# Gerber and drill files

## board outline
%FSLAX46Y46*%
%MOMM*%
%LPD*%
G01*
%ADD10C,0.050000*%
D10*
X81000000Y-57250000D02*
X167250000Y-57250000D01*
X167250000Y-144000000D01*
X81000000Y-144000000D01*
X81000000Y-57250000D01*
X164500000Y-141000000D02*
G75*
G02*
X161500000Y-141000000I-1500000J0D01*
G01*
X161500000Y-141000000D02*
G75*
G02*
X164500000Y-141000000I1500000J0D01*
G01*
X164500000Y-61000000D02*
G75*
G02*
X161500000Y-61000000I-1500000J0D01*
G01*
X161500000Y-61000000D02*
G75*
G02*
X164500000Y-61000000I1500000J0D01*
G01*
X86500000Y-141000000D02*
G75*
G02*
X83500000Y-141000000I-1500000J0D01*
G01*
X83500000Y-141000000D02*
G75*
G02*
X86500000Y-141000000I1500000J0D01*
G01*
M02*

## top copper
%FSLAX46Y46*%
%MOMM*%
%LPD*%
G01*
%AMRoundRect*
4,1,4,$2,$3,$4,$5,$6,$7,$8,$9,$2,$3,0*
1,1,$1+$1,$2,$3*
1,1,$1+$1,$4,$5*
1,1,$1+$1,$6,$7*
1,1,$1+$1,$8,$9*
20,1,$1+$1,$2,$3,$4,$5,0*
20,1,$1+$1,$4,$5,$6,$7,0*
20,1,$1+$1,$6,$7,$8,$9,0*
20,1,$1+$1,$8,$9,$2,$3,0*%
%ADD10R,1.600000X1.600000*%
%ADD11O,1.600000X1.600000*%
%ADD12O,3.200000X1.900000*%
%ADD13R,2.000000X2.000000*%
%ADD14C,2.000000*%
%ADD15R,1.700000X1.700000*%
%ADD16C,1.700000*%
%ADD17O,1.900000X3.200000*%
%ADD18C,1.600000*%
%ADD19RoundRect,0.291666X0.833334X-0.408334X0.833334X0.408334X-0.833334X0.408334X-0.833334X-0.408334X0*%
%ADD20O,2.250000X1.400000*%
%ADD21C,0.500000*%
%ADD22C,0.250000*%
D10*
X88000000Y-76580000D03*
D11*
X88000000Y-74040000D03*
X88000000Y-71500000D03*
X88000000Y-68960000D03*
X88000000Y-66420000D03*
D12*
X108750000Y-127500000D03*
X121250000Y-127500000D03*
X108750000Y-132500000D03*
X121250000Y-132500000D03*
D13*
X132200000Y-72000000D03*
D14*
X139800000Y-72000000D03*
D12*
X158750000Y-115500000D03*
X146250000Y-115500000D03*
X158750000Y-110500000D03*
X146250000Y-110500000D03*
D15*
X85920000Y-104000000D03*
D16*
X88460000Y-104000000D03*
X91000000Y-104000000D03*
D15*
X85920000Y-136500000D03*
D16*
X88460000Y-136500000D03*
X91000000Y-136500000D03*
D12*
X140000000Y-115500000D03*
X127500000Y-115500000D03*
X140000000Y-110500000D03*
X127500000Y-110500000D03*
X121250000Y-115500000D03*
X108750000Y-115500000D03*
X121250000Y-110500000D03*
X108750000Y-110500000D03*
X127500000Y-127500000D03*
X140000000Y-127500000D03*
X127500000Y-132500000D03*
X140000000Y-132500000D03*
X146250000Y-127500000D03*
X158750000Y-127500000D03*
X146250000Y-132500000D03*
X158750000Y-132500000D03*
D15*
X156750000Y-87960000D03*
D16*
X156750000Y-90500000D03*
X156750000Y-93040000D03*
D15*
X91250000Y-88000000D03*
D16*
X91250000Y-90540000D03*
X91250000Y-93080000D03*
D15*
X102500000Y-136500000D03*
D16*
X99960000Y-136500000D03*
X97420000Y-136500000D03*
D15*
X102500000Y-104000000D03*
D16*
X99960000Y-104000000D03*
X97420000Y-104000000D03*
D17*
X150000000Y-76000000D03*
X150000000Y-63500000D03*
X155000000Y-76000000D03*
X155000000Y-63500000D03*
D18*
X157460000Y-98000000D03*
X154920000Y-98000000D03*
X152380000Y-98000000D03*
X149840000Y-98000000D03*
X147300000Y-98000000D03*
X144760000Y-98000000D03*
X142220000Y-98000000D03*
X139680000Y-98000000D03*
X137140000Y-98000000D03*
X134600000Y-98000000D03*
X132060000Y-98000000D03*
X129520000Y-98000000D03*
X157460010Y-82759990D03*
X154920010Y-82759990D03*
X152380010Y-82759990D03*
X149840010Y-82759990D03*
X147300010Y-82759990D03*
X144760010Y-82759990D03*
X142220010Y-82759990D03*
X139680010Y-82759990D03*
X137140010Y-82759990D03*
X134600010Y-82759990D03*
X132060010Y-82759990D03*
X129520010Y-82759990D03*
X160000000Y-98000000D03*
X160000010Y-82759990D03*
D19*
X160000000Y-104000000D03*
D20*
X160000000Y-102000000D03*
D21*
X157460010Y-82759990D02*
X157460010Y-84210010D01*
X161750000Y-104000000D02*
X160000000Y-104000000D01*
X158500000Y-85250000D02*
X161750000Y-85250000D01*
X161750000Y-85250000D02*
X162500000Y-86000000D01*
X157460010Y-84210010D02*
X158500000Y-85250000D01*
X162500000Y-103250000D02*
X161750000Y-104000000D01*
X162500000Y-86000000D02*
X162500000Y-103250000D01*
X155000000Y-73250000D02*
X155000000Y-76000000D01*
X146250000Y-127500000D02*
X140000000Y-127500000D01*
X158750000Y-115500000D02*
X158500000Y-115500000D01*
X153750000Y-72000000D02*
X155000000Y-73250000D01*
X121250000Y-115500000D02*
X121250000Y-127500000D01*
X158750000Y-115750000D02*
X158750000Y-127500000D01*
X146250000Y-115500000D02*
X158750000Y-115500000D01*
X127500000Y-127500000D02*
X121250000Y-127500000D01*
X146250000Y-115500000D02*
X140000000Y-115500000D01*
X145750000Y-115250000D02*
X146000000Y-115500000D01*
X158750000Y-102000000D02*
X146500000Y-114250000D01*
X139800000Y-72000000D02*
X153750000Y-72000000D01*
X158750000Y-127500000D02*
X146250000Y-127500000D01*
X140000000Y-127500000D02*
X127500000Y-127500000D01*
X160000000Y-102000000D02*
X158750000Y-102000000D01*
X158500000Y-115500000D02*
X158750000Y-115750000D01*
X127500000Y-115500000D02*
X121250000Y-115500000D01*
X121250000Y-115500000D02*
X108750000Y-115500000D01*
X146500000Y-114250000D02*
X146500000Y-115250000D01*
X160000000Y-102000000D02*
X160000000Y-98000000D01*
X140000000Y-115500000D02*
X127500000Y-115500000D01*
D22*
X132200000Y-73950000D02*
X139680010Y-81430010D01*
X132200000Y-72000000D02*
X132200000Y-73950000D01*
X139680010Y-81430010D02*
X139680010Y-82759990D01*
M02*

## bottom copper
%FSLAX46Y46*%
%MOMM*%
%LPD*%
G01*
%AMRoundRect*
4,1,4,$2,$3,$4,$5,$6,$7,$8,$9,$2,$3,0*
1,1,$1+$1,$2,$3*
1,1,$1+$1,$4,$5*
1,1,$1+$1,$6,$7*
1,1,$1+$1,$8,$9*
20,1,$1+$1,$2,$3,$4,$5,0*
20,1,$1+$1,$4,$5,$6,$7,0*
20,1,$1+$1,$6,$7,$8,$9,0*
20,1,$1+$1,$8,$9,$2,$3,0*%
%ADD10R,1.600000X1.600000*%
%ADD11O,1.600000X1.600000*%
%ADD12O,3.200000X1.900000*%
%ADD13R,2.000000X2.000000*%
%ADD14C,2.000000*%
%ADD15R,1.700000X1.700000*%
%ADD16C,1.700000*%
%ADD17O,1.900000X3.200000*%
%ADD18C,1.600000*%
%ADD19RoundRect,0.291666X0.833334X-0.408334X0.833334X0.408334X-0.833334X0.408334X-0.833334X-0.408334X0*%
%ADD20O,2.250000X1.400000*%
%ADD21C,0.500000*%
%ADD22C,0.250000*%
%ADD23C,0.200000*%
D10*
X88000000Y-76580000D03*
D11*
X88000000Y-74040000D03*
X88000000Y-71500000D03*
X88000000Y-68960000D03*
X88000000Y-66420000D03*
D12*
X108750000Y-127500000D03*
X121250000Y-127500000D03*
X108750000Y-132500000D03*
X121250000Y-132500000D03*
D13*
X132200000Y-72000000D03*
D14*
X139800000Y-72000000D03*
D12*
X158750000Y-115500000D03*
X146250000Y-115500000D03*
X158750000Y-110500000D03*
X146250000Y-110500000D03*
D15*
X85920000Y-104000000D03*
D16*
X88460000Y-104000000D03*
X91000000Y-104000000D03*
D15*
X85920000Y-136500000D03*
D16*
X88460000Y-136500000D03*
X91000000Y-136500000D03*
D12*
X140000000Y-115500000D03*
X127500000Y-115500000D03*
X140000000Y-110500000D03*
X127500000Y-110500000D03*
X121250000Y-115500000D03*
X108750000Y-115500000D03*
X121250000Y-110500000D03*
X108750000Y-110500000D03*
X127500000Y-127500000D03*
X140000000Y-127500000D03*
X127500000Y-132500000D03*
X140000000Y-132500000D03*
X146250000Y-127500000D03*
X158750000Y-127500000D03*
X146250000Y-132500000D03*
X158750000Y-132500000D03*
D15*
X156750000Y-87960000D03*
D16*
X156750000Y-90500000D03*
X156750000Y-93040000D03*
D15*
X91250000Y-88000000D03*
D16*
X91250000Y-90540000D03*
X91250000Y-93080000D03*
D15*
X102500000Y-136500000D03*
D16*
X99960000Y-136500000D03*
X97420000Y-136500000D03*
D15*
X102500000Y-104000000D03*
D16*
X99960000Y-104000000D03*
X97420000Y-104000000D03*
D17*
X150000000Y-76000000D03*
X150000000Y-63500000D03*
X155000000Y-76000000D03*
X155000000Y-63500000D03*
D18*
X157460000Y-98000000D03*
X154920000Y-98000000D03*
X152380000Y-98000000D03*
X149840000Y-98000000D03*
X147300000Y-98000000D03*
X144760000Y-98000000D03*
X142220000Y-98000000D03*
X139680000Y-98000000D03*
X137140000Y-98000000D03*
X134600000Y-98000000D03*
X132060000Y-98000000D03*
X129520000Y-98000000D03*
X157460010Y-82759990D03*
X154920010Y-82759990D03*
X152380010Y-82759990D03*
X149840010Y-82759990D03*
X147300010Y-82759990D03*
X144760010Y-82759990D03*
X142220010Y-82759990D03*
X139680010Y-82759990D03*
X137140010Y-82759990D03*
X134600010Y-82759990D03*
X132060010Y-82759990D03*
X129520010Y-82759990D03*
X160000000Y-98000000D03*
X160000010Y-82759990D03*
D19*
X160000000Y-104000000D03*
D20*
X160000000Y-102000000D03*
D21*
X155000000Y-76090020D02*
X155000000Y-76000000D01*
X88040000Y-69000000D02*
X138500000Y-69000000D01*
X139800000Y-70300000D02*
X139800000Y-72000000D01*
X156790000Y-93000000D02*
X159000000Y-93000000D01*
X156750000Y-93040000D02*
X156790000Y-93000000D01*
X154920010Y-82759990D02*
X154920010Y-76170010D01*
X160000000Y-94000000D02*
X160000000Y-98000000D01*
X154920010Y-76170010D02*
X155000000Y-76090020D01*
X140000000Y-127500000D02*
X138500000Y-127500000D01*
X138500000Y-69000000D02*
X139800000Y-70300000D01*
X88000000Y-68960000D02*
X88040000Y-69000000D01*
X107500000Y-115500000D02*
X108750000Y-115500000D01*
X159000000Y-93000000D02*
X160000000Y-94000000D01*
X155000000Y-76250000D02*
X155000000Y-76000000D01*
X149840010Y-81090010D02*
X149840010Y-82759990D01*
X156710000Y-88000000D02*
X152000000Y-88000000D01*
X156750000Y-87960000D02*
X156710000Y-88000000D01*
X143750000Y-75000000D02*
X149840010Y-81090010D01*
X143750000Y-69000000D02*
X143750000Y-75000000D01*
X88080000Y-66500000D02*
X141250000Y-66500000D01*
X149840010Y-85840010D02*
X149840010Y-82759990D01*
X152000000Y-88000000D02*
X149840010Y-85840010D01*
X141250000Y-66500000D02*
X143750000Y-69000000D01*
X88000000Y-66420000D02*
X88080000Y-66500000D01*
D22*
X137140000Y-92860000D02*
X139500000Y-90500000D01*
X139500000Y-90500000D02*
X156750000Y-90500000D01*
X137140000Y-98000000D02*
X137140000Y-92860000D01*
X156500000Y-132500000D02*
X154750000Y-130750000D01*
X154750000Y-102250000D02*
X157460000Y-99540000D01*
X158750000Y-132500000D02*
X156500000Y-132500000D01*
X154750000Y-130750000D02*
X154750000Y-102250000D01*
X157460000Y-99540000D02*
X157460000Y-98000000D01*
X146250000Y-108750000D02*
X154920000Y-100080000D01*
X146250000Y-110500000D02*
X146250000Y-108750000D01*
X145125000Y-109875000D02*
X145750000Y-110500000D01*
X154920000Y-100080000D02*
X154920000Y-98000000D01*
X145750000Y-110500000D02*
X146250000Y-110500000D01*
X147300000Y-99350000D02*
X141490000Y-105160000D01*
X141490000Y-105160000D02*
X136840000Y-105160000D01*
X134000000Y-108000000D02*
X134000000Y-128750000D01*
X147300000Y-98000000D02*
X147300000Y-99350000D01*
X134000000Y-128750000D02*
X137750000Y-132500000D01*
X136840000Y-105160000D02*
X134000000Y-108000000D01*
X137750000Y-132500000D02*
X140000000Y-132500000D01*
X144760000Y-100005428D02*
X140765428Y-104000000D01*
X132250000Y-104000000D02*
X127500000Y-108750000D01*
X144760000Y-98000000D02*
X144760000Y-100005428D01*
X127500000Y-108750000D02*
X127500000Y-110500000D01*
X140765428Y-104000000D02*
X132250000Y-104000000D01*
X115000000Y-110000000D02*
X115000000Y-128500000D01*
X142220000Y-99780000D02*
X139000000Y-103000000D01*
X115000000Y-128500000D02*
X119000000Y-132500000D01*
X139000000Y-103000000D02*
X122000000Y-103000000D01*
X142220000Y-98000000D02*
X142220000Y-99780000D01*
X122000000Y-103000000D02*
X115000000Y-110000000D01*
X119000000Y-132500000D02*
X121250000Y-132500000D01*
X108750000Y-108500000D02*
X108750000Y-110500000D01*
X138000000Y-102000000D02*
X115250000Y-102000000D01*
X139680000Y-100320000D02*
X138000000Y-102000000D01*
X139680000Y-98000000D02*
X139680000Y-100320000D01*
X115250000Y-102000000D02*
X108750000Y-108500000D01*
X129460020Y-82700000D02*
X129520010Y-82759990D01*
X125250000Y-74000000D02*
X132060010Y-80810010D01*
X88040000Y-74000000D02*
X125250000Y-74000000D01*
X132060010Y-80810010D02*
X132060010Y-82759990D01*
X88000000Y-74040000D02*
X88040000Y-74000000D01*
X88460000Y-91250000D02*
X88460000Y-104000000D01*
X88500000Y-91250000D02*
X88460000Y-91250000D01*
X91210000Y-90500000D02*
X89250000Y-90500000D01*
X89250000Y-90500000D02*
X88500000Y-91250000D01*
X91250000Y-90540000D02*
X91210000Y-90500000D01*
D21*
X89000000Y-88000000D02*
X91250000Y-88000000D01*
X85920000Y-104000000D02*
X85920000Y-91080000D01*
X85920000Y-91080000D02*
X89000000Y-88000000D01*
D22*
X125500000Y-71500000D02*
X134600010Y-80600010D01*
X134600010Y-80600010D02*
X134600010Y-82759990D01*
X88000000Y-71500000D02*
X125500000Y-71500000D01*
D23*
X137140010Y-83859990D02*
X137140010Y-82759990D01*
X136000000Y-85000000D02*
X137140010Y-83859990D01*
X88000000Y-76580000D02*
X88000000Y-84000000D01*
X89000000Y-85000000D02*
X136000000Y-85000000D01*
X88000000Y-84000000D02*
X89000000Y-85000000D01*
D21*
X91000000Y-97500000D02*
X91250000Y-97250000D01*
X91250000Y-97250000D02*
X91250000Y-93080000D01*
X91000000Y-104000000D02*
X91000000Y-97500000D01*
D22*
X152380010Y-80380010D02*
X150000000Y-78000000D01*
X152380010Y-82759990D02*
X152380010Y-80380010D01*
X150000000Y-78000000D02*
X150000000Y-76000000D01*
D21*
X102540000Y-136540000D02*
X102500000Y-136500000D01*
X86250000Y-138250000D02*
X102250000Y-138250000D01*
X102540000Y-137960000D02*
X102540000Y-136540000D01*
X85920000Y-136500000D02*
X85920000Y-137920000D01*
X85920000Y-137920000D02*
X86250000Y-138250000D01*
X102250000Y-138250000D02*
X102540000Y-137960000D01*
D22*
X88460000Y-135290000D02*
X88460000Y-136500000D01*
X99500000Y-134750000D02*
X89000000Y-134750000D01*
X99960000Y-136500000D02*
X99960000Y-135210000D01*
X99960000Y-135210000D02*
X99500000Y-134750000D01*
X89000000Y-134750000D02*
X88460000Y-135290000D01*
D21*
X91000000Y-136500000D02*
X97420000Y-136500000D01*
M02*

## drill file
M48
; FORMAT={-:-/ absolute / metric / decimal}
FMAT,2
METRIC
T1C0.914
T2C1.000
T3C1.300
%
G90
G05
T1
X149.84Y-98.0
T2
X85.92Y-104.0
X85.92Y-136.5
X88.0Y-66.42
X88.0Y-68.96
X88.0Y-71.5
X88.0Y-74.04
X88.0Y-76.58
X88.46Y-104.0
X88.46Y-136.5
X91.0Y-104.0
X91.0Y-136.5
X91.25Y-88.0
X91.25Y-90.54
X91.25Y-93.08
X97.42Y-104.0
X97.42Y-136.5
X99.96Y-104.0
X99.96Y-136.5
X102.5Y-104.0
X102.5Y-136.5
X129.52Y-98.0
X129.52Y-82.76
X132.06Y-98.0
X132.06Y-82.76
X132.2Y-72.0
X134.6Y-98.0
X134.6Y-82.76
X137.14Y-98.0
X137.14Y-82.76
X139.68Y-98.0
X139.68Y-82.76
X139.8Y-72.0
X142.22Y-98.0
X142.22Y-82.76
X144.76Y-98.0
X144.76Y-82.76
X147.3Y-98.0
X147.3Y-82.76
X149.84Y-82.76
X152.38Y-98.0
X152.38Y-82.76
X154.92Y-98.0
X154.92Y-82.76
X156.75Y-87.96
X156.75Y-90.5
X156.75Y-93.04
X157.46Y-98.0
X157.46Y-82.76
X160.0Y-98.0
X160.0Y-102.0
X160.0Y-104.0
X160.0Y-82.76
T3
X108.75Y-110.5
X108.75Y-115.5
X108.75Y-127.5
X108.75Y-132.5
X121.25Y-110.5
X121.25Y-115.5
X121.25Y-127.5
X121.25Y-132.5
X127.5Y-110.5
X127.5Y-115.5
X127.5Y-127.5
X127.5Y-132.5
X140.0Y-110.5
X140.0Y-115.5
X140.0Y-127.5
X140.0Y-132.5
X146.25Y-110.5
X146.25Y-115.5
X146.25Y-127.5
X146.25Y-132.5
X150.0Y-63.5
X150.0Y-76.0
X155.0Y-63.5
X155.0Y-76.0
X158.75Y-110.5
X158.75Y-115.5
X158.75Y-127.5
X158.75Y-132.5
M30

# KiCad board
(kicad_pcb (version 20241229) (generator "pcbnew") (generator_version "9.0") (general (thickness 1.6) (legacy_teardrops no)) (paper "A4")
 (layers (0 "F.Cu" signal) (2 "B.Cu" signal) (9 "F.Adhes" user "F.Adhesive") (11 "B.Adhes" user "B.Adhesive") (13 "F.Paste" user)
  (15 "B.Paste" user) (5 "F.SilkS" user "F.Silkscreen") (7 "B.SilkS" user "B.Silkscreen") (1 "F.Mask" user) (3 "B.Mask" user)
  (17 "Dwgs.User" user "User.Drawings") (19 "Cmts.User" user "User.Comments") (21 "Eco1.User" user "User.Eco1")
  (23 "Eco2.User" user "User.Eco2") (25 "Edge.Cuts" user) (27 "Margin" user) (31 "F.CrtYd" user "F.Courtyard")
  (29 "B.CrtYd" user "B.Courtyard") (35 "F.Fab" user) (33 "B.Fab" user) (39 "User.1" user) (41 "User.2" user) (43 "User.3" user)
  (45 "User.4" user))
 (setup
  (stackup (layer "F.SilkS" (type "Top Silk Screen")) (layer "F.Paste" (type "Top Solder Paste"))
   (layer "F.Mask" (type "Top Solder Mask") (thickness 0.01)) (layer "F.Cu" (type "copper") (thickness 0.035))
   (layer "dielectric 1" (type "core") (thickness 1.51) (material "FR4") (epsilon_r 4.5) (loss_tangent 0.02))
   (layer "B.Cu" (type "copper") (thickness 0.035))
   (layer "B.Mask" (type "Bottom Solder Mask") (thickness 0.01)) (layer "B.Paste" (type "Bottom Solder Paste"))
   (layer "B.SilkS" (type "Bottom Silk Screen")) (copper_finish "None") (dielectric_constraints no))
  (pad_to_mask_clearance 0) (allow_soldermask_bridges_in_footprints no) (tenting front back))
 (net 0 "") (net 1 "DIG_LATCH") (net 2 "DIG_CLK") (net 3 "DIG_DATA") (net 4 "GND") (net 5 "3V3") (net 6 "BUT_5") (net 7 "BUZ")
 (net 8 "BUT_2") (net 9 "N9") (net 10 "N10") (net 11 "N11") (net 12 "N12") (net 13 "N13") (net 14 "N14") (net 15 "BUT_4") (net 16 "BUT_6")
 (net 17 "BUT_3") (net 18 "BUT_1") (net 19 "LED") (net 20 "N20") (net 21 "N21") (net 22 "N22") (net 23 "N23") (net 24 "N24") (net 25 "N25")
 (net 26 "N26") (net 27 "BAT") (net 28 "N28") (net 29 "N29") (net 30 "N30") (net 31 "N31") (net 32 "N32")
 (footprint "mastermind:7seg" (layer "F.Cu") (at 94.5 68)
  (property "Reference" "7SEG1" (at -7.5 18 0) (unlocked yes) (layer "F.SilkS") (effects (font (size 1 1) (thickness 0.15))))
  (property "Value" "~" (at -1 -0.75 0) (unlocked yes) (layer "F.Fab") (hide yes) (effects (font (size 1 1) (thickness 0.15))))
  (pad "1" thru_hole rect (at -6.5 8.58 180) (size 1.6 1.6) (drill 1) (layers "*.Cu" "*.Mask") (remove_unused_layers no) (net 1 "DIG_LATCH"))
  (pad "2" thru_hole oval (at -6.5 6.04 180) (size 1.6 1.6) (drill 1) (layers "*.Cu" "*.Mask") (remove_unused_layers no) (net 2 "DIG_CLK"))
  (pad "3" thru_hole oval (at -6.5 3.5 180) (size 1.6 1.6) (drill 1) (layers "*.Cu" "*.Mask") (remove_unused_layers no) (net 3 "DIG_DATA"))
  (pad "4" thru_hole oval (at -6.5 0.96 180) (size 1.6 1.6) (drill 1) (layers "*.Cu" "*.Mask") (remove_unused_layers no) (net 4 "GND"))
  (pad "5" thru_hole oval (at -6.5 -1.58 180) (size 1.6 1.6) (drill 1) (layers "*.Cu" "*.Mask") (remove_unused_layers no) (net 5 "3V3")))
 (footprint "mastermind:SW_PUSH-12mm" (layer "F.Cu") (at 108.75 127.5)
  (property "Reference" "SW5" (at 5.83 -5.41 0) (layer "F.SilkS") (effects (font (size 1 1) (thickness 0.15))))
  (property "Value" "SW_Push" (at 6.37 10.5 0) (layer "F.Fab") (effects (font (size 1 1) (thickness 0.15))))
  (pad "1" thru_hole oval (at 0 0) (size 3.2 1.9) (drill 1.3) (layers "*.Cu" "*.Mask") (remove_unused_layers no) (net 4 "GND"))
  (pad "1" thru_hole oval (at 12.5 0) (size 3.2 1.9) (drill 1.3) (layers "*.Cu" "*.Mask") (remove_unused_layers no) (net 4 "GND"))
  (pad "2" thru_hole oval (at 0 5) (size 3.2 1.9) (drill 1.3) (layers "*.Cu" "*.Mask") (remove_unused_layers no) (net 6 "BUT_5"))
  (pad "2" thru_hole oval (at 12.5 5) (size 3.2 1.9) (drill 1.3) (layers "*.Cu" "*.Mask") (remove_unused_layers no) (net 6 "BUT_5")))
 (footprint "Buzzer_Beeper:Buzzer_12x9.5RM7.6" (layer "F.Cu") (at 132.2 72)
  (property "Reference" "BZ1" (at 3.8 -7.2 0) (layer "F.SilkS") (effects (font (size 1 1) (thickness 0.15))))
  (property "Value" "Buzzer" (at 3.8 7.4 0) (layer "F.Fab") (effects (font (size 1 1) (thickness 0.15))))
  (pad "1" thru_hole rect (at 0 0) (size 2 2) (drill 1) (layers "*.Cu" "*.Mask") (remove_unused_layers no) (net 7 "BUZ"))
  (pad "2" thru_hole circle (at 7.6 0) (size 2 2) (drill 1) (layers "*.Cu" "*.Mask") (remove_unused_layers no) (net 4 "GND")))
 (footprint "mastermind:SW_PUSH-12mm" (layer "F.Cu") (at 158.75 115.5 180)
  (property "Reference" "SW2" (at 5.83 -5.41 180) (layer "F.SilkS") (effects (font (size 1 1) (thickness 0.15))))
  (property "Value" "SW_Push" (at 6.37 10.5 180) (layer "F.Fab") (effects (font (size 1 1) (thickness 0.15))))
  (pad "1" thru_hole oval (at 0 0 180) (size 3.2 1.9) (drill 1.3) (layers "*.Cu" "*.Mask") (remove_unused_layers no) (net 4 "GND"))
  (pad "1" thru_hole oval (at 12.5 0 180) (size 3.2 1.9) (drill 1.3) (layers "*.Cu" "*.Mask") (remove_unused_layers no) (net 4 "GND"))
  (pad "2" thru_hole oval (at 0 5 180) (size 3.2 1.9) (drill 1.3) (layers "*.Cu" "*.Mask") (remove_unused_layers no) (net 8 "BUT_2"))
  (pad "2" thru_hole oval (at 12.5 5 180) (size 3.2 1.9) (drill 1.3) (layers "*.Cu" "*.Mask") (remove_unused_layers no) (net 8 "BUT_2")))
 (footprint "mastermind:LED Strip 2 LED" (layer "F.Cu") (at 88.17 111.25 90)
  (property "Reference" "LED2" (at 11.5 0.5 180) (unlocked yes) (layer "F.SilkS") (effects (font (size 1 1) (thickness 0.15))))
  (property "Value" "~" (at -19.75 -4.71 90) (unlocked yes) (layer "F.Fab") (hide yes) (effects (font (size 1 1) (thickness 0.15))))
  (pad "1" thru_hole rect (at 7.25 -2.25 90) (size 1.7 1.7) (drill 1) (layers "*.Cu" "*.Mask") (remove_unused_layers no) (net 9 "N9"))
  (pad "2" thru_hole circle (at 7.25 0.29 90) (size 1.7 1.7) (drill 1) (layers "*.Cu" "*.Mask") (remove_unused_layers no) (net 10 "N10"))
  (pad "3" thru_hole circle (at 7.25 2.83 90) (size 1.7 1.7) (drill 1) (layers "*.Cu" "*.Mask") (remove_unused_layers no) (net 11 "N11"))
  (pad "4" thru_hole rect (at -25.25 -2.25 90) (size 1.7 1.7) (drill 1) (layers "*.Cu" "*.Mask") (remove_unused_layers no) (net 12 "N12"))
  (pad "5" thru_hole circle (at -25.25 0.29 90) (size 1.7 1.7) (drill 1) (layers "*.Cu" "*.Mask") (remove_unused_layers no) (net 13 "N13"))
  (pad "6" thru_hole circle (at -25.25 2.83 90) (size 1.7 1.7) (drill 1) (layers "*.Cu" "*.Mask") (remove_unused_layers no) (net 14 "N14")))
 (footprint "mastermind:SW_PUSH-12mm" (layer "F.Cu") (at 140 115.5 180)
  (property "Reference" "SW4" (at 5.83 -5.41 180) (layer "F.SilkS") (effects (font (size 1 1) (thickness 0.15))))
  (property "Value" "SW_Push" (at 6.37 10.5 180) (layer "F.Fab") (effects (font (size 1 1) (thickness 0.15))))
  (pad "1" thru_hole oval (at 0 0 180) (size 3.2 1.9) (drill 1.3) (layers "*.Cu" "*.Mask") (remove_unused_layers no) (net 4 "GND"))
  (pad "1" thru_hole oval (at 12.5 0 180) (size 3.2 1.9) (drill 1.3) (layers "*.Cu" "*.Mask") (remove_unused_layers no) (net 4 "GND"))
  (pad "2" thru_hole oval (at 0 5 180) (size 3.2 1.9) (drill 1.3) (layers "*.Cu" "*.Mask") (remove_unused_layers no) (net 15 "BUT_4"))
  (pad "2" thru_hole oval (at 12.5 5 180) (size 3.2 1.9) (drill 1.3) (layers "*.Cu" "*.Mask") (remove_unused_layers no) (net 15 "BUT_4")))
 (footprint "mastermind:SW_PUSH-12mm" (layer "F.Cu") (at 121.25 115.5 180)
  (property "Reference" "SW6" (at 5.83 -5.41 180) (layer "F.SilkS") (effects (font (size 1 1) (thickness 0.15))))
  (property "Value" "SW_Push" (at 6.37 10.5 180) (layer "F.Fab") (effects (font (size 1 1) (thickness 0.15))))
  (pad "1" thru_hole oval (at 0 0 180) (size 3.2 1.9) (drill 1.3) (layers "*.Cu" "*.Mask") (remove_unused_layers no) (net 4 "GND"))
  (pad "1" thru_hole oval (at 12.5 0 180) (size 3.2 1.9) (drill 1.3) (layers "*.Cu" "*.Mask") (remove_unused_layers no) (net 4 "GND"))
  (pad "2" thru_hole oval (at 0 5 180) (size 3.2 1.9) (drill 1.3) (layers "*.Cu" "*.Mask") (remove_unused_layers no) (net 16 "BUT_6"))
  (pad "2" thru_hole oval (at 12.5 5 180) (size 3.2 1.9) (drill 1.3) (layers "*.Cu" "*.Mask") (remove_unused_layers no) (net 16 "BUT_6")))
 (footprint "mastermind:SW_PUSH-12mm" (layer "F.Cu") (at 127.5 127.5)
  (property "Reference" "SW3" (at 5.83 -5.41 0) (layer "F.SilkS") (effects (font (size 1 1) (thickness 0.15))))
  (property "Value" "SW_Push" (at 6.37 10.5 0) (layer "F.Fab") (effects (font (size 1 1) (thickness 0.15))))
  (pad "1" thru_hole oval (at 0 0) (size 3.2 1.9) (drill 1.3) (layers "*.Cu" "*.Mask") (remove_unused_layers no) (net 4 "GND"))
  (pad "1" thru_hole oval (at 12.5 0) (size 3.2 1.9) (drill 1.3) (layers "*.Cu" "*.Mask") (remove_unused_layers no) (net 4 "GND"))
  (pad "2" thru_hole oval (at 0 5) (size 3.2 1.9) (drill 1.3) (layers "*.Cu" "*.Mask") (remove_unused_layers no) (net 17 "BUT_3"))
  (pad "2" thru_hole oval (at 12.5 5) (size 3.2 1.9) (drill 1.3) (layers "*.Cu" "*.Mask") (remove_unused_layers no) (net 17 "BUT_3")))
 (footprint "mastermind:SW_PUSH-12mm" (layer "F.Cu") (at 146.25 127.5)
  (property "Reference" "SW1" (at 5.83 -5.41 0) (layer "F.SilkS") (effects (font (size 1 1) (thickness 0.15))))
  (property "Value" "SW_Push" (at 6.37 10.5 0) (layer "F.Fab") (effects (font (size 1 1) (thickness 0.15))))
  (pad "1" thru_hole oval (at 0 0) (size 3.2 1.9) (drill 1.3) (layers "*.Cu" "*.Mask") (remove_unused_layers no) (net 4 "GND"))
  (pad "1" thru_hole oval (at 12.5 0) (size 3.2 1.9) (drill 1.3) (layers "*.Cu" "*.Mask") (remove_unused_layers no) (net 4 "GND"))
  (pad "2" thru_hole oval (at 0 5) (size 3.2 1.9) (drill 1.3) (layers "*.Cu" "*.Mask") (remove_unused_layers no) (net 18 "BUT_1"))
  (pad "2" thru_hole oval (at 12.5 5) (size 3.2 1.9) (drill 1.3) (layers "*.Cu" "*.Mask") (remove_unused_layers no) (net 18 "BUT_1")))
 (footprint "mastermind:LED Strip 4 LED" (layer "F.Cu") (at 115.5 90.25)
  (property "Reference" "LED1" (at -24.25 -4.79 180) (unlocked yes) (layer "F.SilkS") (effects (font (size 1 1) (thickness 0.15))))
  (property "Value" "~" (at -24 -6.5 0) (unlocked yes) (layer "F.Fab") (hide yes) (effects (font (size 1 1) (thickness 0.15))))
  (pad "1" thru_hole rect (at 41.25 -2.29) (size 1.7 1.7) (drill 1) (layers "*.Cu" "*.Mask") (remove_unused_layers no) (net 5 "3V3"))
  (pad "2" thru_hole circle (at 41.25 0.25) (size 1.7 1.7) (drill 1) (layers "*.Cu" "*.Mask") (remove_unused_layers no) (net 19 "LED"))
  (pad "3" thru_hole circle (at 41.25 2.79) (size 1.7 1.7) (drill 1) (layers "*.Cu" "*.Mask") (remove_unused_layers no) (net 4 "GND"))
  (pad "4" thru_hole rect (at -24.25 -2.25) (size 1.7 1.7) (drill 1) (layers "*.Cu" "*.Mask") (remove_unused_layers no) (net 9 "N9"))
  (pad "5" thru_hole circle (at -24.25 0.29) (size 1.7 1.7) (drill 1) (layers "*.Cu" "*.Mask") (remove_unused_layers no) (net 10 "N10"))
  (pad "6" thru_hole circle (at -24.25 2.83) (size 1.7 1.7) (drill 1) (layers "*.Cu" "*.Mask") (remove_unused_layers no) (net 11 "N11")))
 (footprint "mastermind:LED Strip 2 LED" (layer "F.Cu") (at 100.25 129.25 -90)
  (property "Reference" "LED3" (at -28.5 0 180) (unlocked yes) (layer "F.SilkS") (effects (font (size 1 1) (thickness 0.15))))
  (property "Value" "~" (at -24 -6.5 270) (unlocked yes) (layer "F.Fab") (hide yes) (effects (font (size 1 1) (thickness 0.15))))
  (pad "1" thru_hole rect (at 7.25 -2.25 270) (size 1.7 1.7) (drill 1) (layers "*.Cu" "*.Mask") (remove_unused_layers no) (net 12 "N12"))
  (pad "2" thru_hole circle (at 7.25 0.29 270) (size 1.7 1.7) (drill 1) (layers "*.Cu" "*.Mask") (remove_unused_layers no) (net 13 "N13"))
  (pad "3" thru_hole circle (at 7.25 2.83 270) (size 1.7 1.7) (drill 1) (layers "*.Cu" "*.Mask") (remove_unused_layers no) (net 14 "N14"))
  (pad "4" thru_hole rect (at -25.25 -2.25 270) (size 1.7 1.7) (drill 1) (layers "*.Cu" "*.Mask") (remove_unused_layers no) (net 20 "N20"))
  (pad "5" thru_hole circle (at -25.25 0.29 270) (size 1.7 1.7) (drill 1) (layers "*.Cu" "*.Mask") (remove_unused_layers no) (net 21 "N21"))
  (pad "6" thru_hole circle (at -25.25 2.83 270) (size 1.7 1.7) (drill 1) (layers "*.Cu" "*.Mask") (remove_unused_layers no) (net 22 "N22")))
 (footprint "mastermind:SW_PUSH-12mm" (layer "F.Cu") (at 150 76 90)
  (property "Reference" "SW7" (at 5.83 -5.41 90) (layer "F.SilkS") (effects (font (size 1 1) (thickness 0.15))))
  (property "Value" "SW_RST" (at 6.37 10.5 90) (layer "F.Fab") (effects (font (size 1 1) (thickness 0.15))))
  (pad "1" thru_hole oval (at 0 0 90) (size 3.2 1.9) (drill 1.3) (layers "*.Cu" "*.Mask") (remove_unused_layers no) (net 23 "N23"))
  (pad "1" thru_hole oval (at 12.5 0 90) (size 3.2 1.9) (drill 1.3) (layers "*.Cu" "*.Mask") (remove_unused_layers no) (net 23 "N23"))
  (pad "2" thru_hole oval (at 0 5 90) (size 3.2 1.9) (drill 1.3) (layers "*.Cu" "*.Mask") (remove_unused_layers no) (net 4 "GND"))
  (pad "2" thru_hole oval (at 12.5 5 90) (size 3.2 1.9) (drill 1.3) (layers "*.Cu" "*.Mask") (remove_unused_layers no) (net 4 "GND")))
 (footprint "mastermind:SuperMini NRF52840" (layer "B.Cu") (at 160 98 90)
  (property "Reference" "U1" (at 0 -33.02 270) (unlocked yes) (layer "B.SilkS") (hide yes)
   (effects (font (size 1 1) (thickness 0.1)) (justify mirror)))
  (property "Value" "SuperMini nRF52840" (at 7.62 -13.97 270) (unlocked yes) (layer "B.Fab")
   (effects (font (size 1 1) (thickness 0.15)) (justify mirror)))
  (pad "1" thru_hole circle (at 0 -2.54 180) (size 1.6 1.6) (drill 1) (layers "*.Cu" "*.Mask") (remove_unused_layers no) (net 18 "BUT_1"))
  (pad "2" thru_hole circle (at 0 -5.08 180) (size 1.6 1.6) (drill 1) (layers "*.Cu" "*.Mask") (remove_unused_layers no) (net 8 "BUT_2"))
  (pad "3" thru_hole circle (at 0 -7.62 180) (size 1.6 1.6) (drill 1) (layers "*.Cu" "*.Mask") (remove_unused_layers no) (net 4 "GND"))
  (pad "4" thru_hole circle (at 0 -10.16) (size 1.6 1.6) (drill 0.9144) (layers "*.Cu" "*.Mask") (remove_unused_layers no) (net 4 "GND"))
  (pad "5" thru_hole circle (at 0 -12.7 180) (size 1.6 1.6) (drill 1) (layers "*.Cu" "*.Mask") (remove_unused_layers no) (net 17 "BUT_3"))
  (pad "6" thru_hole circle (at 0 -15.24 180) (size 1.6 1.6) (drill 1) (layers "*.Cu" "*.Mask") (remove_unused_layers no) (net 15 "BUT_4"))
  (pad "7" thru_hole circle (at 0 -17.78 180) (size 1.6 1.6) (drill 1) (layers "*.Cu" "*.Mask") (remove_unused_layers no) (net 6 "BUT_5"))
  (pad "8" thru_hole circle (at 0 -20.32 180) (size 1.6 1.6) (drill 1) (layers "*.Cu" "*.Mask") (remove_unused_layers no) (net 16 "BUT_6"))
  (pad "9" thru_hole circle (at 0 -22.86 180) (size 1.6 1.6) (drill 1) (layers "*.Cu" "*.Mask") (remove_unused_layers no) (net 19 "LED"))
  (pad "10" thru_hole circle (at 0 -25.4 180) (size 1.6 1.6) (drill 1) (layers "*.Cu" "*.Mask") (remove_unused_layers no) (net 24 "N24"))
  (pad "11" thru_hole circle (at 0 -27.94 180) (size 1.6 1.6) (drill 1) (layers "*.Cu" "*.Mask") (remove_unused_layers no) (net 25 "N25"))
  (pad "12" thru_hole circle (at 0 -30.48 180) (size 1.6 1.6) (drill 1) (layers "*.Cu" "*.Mask") (remove_unused_layers no) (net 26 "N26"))
  (pad "13" thru_hole circle (at 15.24001 -2.53999) (size 1.6 1.6) (drill 1) (layers "*.Cu" "*.Mask") (remove_unused_layers no)
   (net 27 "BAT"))
  (pad "14" thru_hole circle (at 15.24001 -5.07999) (size 1.6 1.6) (drill 1) (layers "*.Cu" "*.Mask") (remove_unused_layers no)
   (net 4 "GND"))
  (pad "15" thru_hole circle (at 15.24001 -7.61999) (size 1.6 1.6) (drill 1) (layers "*.Cu" "*.Mask") (remove_unused_layers no)
   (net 23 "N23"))
  (pad "16" thru_hole circle (at 15.24001 -10.15999) (size 1.6 1.6) (drill 1) (layers "*.Cu" "*.Mask") (remove_unused_layers no)
   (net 5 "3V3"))
  (pad "17" thru_hole circle (at 15.24001 -12.69999) (size 1.6 1.6) (drill 1) (layers "*.Cu" "*.Mask") (remove_unused_layers no)
   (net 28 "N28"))
  (pad "18" thru_hole circle (at 15.24001 -15.23999) (size 1.6 1.6) (drill 1) (layers "*.Cu" "*.Mask") (remove_unused_layers no)
   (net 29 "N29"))
  (pad "19" thru_hole circle (at 15.24001 -17.77999) (size 1.6 1.6) (drill 1) (layers "*.Cu" "*.Mask") (remove_unused_layers no)
   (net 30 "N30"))
  (pad "20" thru_hole circle (at 15.24001 -20.31999) (size 1.6 1.6) (drill 1) (layers "*.Cu" "*.Mask") (remove_unused_layers no)
   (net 7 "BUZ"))
  (pad "21" thru_hole circle (at 15.24001 -22.85999) (size 1.6 1.6) (drill 1) (layers "*.Cu" "*.Mask") (remove_unused_layers no)
   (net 1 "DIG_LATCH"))
  (pad "22" thru_hole circle (at 15.24001 -25.39999) (size 1.6 1.6) (drill 1) (layers "*.Cu" "*.Mask") (remove_unused_layers no)
   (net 3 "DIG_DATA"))
  (pad "23" thru_hole circle (at 15.24001 -27.93999) (size 1.6 1.6) (drill 1) (layers "*.Cu" "*.Mask") (remove_unused_layers no)
   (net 2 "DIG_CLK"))
  (pad "24" thru_hole circle (at 15.24001 -30.47999 180) (size 1.6 1.6) (drill 1) (layers "*.Cu" "*.Mask") (remove_unused_layers no)
   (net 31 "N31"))
  (pad "28" thru_hole circle (at 0 0 180) (size 1.6 1.6) (drill 1) (layers "*.Cu" "*.Mask") (remove_unused_layers no) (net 4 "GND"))
  (pad "29" thru_hole circle (at 15.24001 0.00001) (size 1.6 1.6) (drill 1) (layers "*.Cu" "*.Mask") (remove_unused_layers no)
   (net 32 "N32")))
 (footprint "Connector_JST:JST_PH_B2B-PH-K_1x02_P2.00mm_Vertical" (layer "B.Cu") (at 160 104 90)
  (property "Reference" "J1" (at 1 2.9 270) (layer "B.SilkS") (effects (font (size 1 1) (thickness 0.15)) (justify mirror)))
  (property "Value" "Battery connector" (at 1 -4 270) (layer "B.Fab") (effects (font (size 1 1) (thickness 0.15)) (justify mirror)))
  (pad "1" thru_hole roundrect (at 0 0 90) (size 1.4 2.25) (drill 1) (layers "*.Cu" "*.Mask") (remove_unused_layers no)
   (roundrect_rratio 0.208333) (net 27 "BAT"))
  (pad "2" thru_hole oval (at 2 0 90) (size 1.4 2.25) (drill 1) (layers "*.Cu" "*.Mask") (remove_unused_layers no) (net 4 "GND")))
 (gr_rect (start 81 57.25) (end 167.25 144) (stroke (width 0.05) (type default)) (fill no) (layer "Edge.Cuts"))
 (gr_circle (center 163 141) (end 164.5 141) (stroke (width 0.05) (type solid)) (fill no) (layer "Edge.Cuts"))
 (gr_circle (center 163 61) (end 164.5 61) (stroke (width 0.05) (type solid)) (fill no) (layer "Edge.Cuts"))
 (gr_circle (center 85 141) (end 86.5 141) (stroke (width 0.05) (type solid)) (fill no) (layer "Edge.Cuts"))
 (segment (start 157.46001 82.75999) (end 157.46001 84.21001) (width 0.5) (layer "F.Cu") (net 27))
 (segment (start 161.75 104) (end 160 104) (width 0.5) (layer "F.Cu") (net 27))
 (segment (start 158.5 85.25) (end 161.75 85.25) (width 0.5) (layer "F.Cu") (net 27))
 (segment (start 161.75 85.25) (end 162.5 86) (width 0.5) (layer "F.Cu") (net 27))
 (segment (start 157.46001 84.21001) (end 158.5 85.25) (width 0.5) (layer "F.Cu") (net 27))
 (segment (start 162.5 103.25) (end 161.75 104) (width 0.5) (layer "F.Cu") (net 27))
 (segment (start 162.5 86) (end 162.5 103.25) (width 0.5) (layer "F.Cu") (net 27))
 (segment (start 155 73.25) (end 155 76) (width 0.5) (layer "F.Cu") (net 4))
 (segment (start 146.25 127.5) (end 140 127.5) (width 0.5) (layer "F.Cu") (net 4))
 (segment (start 158.75 115.5) (end 158.5 115.5) (width 0.5) (layer "F.Cu") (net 4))
 (segment (start 153.75 72) (end 155 73.25) (width 0.5) (layer "F.Cu") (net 4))
 (segment (start 121.25 115.5) (end 121.25 127.5) (width 0.5) (layer "F.Cu") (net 4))
 (segment (start 158.75 115.75) (end 158.75 127.5) (width 0.5) (layer "F.Cu") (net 4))
 (segment (start 146.25 115.5) (end 158.75 115.5) (width 0.5) (layer "F.Cu") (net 4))
 (segment (start 127.5 127.5) (end 121.25 127.5) (width 0.5) (layer "F.Cu") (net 4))
 (segment (start 146.25 115.5) (end 140 115.5) (width 0.5) (layer "F.Cu") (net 4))
 (segment (start 145.75 115.25) (end 146 115.5) (width 0.5) (layer "F.Cu") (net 4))
 (segment (start 158.75 102) (end 146.5 114.25) (width 0.5) (layer "F.Cu") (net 4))
 (segment (start 139.8 72) (end 153.75 72) (width 0.5) (layer "F.Cu") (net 4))
 (segment (start 158.75 127.5) (end 146.25 127.5) (width 0.5) (layer "F.Cu") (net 4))
 (segment (start 140 127.5) (end 127.5 127.5) (width 0.5) (layer "F.Cu") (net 4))
 (segment (start 160 102) (end 158.75 102) (width 0.5) (layer "F.Cu") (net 4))
 (segment (start 158.5 115.5) (end 158.75 115.75) (width 0.5) (layer "F.Cu") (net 4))
 (segment (start 127.5 115.5) (end 121.25 115.5) (width 0.5) (layer "F.Cu") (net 4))
 (segment (start 121.25 115.5) (end 108.75 115.5) (width 0.5) (layer "F.Cu") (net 4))
 (segment (start 146.5 114.25) (end 146.5 115.25) (width 0.5) (layer "F.Cu") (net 4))
 (segment (start 160 102) (end 160 98) (width 0.5) (layer "F.Cu") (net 4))
 (segment (start 140 115.5) (end 127.5 115.5) (width 0.5) (layer "F.Cu") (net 4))
 (segment (start 155 76.09002) (end 155 76) (width 0.5) (layer "B.Cu") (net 4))
 (segment (start 88.04 69) (end 138.5 69) (width 0.5) (layer "B.Cu") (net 4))
 (segment (start 139.8 70.3) (end 139.8 72) (width 0.5) (layer "B.Cu") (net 4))
 (segment (start 156.79 93) (end 159 93) (width 0.5) (layer "B.Cu") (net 4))
 (segment (start 156.75 93.04) (end 156.79 93) (width 0.5) (layer "B.Cu") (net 4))
 (segment (start 154.92001 82.75999) (end 154.92001 76.17001) (width 0.5) (layer "B.Cu") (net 4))
 (segment (start 160 94) (end 160 98) (width 0.5) (layer "B.Cu") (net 4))
 (segment (start 154.92001 76.17001) (end 155 76.09002) (width 0.5) (layer "B.Cu") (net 4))
 (segment (start 140 127.5) (end 138.5 127.5) (width 0.5) (layer "B.Cu") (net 4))
 (segment (start 138.5 69) (end 139.8 70.3) (width 0.5) (layer "B.Cu") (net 4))
 (segment (start 88 68.96) (end 88.04 69) (width 0.5) (layer "B.Cu") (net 4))
 (segment (start 107.5 115.5) (end 108.75 115.5) (width 0.5) (layer "B.Cu") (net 4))
 (segment (start 159 93) (end 160 94) (width 0.5) (layer "B.Cu") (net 4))
 (segment (start 155 76.25) (end 155 76) (width 0.5) (layer "B.Cu") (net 4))
 (segment (start 149.84001 81.09001) (end 149.84001 82.75999) (width 0.5) (layer "B.Cu") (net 5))
 (segment (start 156.71 88) (end 152 88) (width 0.5) (layer "B.Cu") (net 5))
 (segment (start 156.75 87.96) (end 156.71 88) (width 0.5) (layer "B.Cu") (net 5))
 (segment (start 143.75 75) (end 149.84001 81.09001) (width 0.5) (layer "B.Cu") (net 5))
 (segment (start 143.75 69) (end 143.75 75) (width 0.5) (layer "B.Cu") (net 5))
 (segment (start 88.08 66.5) (end 141.25 66.5) (width 0.5) (layer "B.Cu") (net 5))
 (segment (start 149.84001 85.84001) (end 149.84001 82.75999) (width 0.5) (layer "B.Cu") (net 5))
 (segment (start 152 88) (end 149.84001 85.84001) (width 0.5) (layer "B.Cu") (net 5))
 (segment (start 141.25 66.5) (end 143.75 69) (width 0.5) (layer "B.Cu") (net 5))
 (segment (start 88 66.42) (end 88.08 66.5) (width 0.5) (layer "B.Cu") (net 5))
 (segment (start 137.14 92.86) (end 139.5 90.5) (width 0.25) (layer "B.Cu") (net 19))
 (segment (start 139.5 90.5) (end 156.75 90.5) (width 0.25) (layer "B.Cu") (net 19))
 (segment (start 137.14 98) (end 137.14 92.86) (width 0.25) (layer "B.Cu") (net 19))
 (segment (start 156.5 132.5) (end 154.75 130.75) (width 0.25) (layer "B.Cu") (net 18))
 (segment (start 154.75 102.25) (end 157.46 99.54) (width 0.25) (layer "B.Cu") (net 18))
 (segment (start 158.75 132.5) (end 156.5 132.5) (width 0.25) (layer "B.Cu") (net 18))
 (segment (start 154.75 130.75) (end 154.75 102.25) (width 0.25) (layer "B.Cu") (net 18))
 (segment (start 157.46 99.54) (end 157.46 98) (width 0.25) (layer "B.Cu") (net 18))
 (segment (start 146.25 108.75) (end 154.92 100.08) (width 0.25) (layer "B.Cu") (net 8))
 (segment (start 146.25 110.5) (end 146.25 108.75) (width 0.25) (layer "B.Cu") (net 8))
 (segment (start 145.125 109.875) (end 145.75 110.5) (width 0.25) (layer "B.Cu") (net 8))
 (segment (start 154.92 100.08) (end 154.92 98) (width 0.25) (layer "B.Cu") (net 8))
 (segment (start 145.75 110.5) (end 146.25 110.5) (width 0.25) (layer "B.Cu") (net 8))
 (segment (start 147.3 99.35) (end 141.49 105.16) (width 0.25) (layer "B.Cu") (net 17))
 (segment (start 141.49 105.16) (end 136.84 105.16) (width 0.25) (layer "B.Cu") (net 17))
 (segment (start 134 108) (end 134 128.75) (width 0.25) (layer "B.Cu") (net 17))
 (segment (start 147.3 98) (end 147.3 99.35) (width 0.25) (layer "B.Cu") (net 17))
 (segment (start 134 128.75) (end 137.75 132.5) (width 0.25) (layer "B.Cu") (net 17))
 (segment (start 136.84 105.16) (end 134 108) (width 0.25) (layer "B.Cu") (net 17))
 (segment (start 137.75 132.5) (end 140 132.5) (width 0.25) (layer "B.Cu") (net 17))
 (segment (start 144.76 100.005428) (end 140.765428 104) (width 0.25) (layer "B.Cu") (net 15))
 (segment (start 132.25 104) (end 127.5 108.75) (width 0.25) (layer "B.Cu") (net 15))
 (segment (start 144.76 98) (end 144.76 100.005428) (width 0.25) (layer "B.Cu") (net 15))
 (segment (start 127.5 108.75) (end 127.5 110.5) (width 0.25) (layer "B.Cu") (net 15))
 (segment (start 140.765428 104) (end 132.25 104) (width 0.25) (layer "B.Cu") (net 15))
 (segment (start 115 110) (end 115 128.5) (width 0.25) (layer "B.Cu") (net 6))
 (segment (start 142.22 99.78) (end 139 103) (width 0.25) (layer "B.Cu") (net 6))
 (segment (start 115 128.5) (end 119 132.5) (width 0.25) (layer "B.Cu") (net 6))
 (segment (start 139 103) (end 122 103) (width 0.25) (layer "B.Cu") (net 6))
 (segment (start 142.22 98) (end 142.22 99.78) (width 0.25) (layer "B.Cu") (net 6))
 (segment (start 122 103) (end 115 110) (width 0.25) (layer "B.Cu") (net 6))
 (segment (start 119 132.5) (end 121.25 132.5) (width 0.25) (layer "B.Cu") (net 6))
 (segment (start 108.75 108.5) (end 108.75 110.5) (width 0.25) (layer "B.Cu") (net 16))
 (segment (start 138 102) (end 115.25 102) (width 0.25) (layer "B.Cu") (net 16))
 (segment (start 139.68 100.32) (end 138 102) (width 0.25) (layer "B.Cu") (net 16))
 (segment (start 139.68 98) (end 139.68 100.32) (width 0.25) (layer "B.Cu") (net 16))
 (segment (start 115.25 102) (end 108.75 108.5) (width 0.25) (layer "B.Cu") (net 16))
 (segment (start 129.46002 82.7) (end 129.52001 82.75999) (width 0.25) (layer "B.Cu") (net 31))
 (segment (start 132.2 73.95) (end 139.68001 81.43001) (width 0.25) (layer "F.Cu") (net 7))
 (segment (start 132.2 72) (end 132.2 73.95) (width 0.25) (layer "F.Cu") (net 7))
 (segment (start 139.68001 81.43001) (end 139.68001 82.75999) (width 0.25) (layer "F.Cu") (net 7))
 (segment (start 125.25 74) (end 132.06001 80.81001) (width 0.25) (layer "B.Cu") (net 2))
 (segment (start 88.04 74) (end 125.25 74) (width 0.25) (layer "B.Cu") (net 2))
 (segment (start 132.06001 80.81001) (end 132.06001 82.75999) (width 0.25) (layer "B.Cu") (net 2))
 (segment (start 88 74.04) (end 88.04 74) (width 0.25) (layer "B.Cu") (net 2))
 (segment (start 88.46 91.25) (end 88.46 104) (width 0.25) (layer "B.Cu") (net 10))
 (segment (start 88.5 91.25) (end 88.46 91.25) (width 0.25) (layer "B.Cu") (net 10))
 (segment (start 91.21 90.5) (end 89.25 90.5) (width 0.25) (layer "B.Cu") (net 10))
 (segment (start 89.25 90.5) (end 88.5 91.25) (width 0.25) (layer "B.Cu") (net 10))
 (segment (start 91.25 90.54) (end 91.21 90.5) (width 0.25) (layer "B.Cu") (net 10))
 (segment (start 89 88) (end 91.25 88) (width 0.5) (layer "B.Cu") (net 9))
 (segment (start 85.92 104) (end 85.92 91.08) (width 0.5) (layer "B.Cu") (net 9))
 (segment (start 85.92 91.08) (end 89 88) (width 0.5) (layer "B.Cu") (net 9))
 (segment (start 125.5 71.5) (end 134.60001 80.60001) (width 0.25) (layer "B.Cu") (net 3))
 (segment (start 134.60001 80.60001) (end 134.60001 82.75999) (width 0.25) (layer "B.Cu") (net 3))
 (segment (start 88 71.5) (end 125.5 71.5) (width 0.25) (layer "B.Cu") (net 3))
 (segment (start 137.14001 83.85999) (end 137.14001 82.75999) (width 0.2) (layer "B.Cu") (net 1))
 (segment (start 136 85) (end 137.14001 83.85999) (width 0.2) (layer "B.Cu") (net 1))
 (segment (start 88 76.58) (end 88 84) (width 0.2) (layer "B.Cu") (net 1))
 (segment (start 89 85) (end 136 85) (width 0.2) (layer "B.Cu") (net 1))
 (segment (start 88 84) (end 89 85) (width 0.2) (layer "B.Cu") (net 1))
 (segment (start 91 97.5) (end 91.25 97.25) (width 0.5) (layer "B.Cu") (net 11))
 (segment (start 91.25 97.25) (end 91.25 93.08) (width 0.5) (layer "B.Cu") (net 11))
 (segment (start 91 104) (end 91 97.5) (width 0.5) (layer "B.Cu") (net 11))
 (segment (start 152.38001 80.38001) (end 150 78) (width 0.25) (layer "B.Cu") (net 23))
 (segment (start 152.38001 82.75999) (end 152.38001 80.38001) (width 0.25) (layer "B.Cu") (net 23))
 (segment (start 150 78) (end 150 76) (width 0.25) (layer "B.Cu") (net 23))
 (segment (start 102.54 136.54) (end 102.5 136.5) (width 0.5) (layer "B.Cu") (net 12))
 (segment (start 86.25 138.25) (end 102.25 138.25) (width 0.5) (layer "B.Cu") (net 12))
 (segment (start 102.54 137.96) (end 102.54 136.54) (width 0.5) (layer "B.Cu") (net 12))
 (segment (start 85.92 136.5) (end 85.92 137.92) (width 0.5) (layer "B.Cu") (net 12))
 (segment (start 85.92 137.92) (end 86.25 138.25) (width 0.5) (layer "B.Cu") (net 12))
 (segment (start 102.25 138.25) (end 102.54 137.96) (width 0.5) (layer "B.Cu") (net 12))
 (segment (start 88.46 135.29) (end 88.46 136.5) (width 0.25) (layer "B.Cu") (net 13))
 (segment (start 99.5 134.75) (end 89 134.75) (width 0.25) (layer "B.Cu") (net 13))
 (segment (start 99.96 136.5) (end 99.96 135.21) (width 0.25) (layer "B.Cu") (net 13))
 (segment (start 99.96 135.21) (end 99.5 134.75) (width 0.25) (layer "B.Cu") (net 13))
 (segment (start 89 134.75) (end 88.46 135.29) (width 0.25) (layer "B.Cu") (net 13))
 (segment (start 91 136.5) (end 97.42 136.5) (width 0.5) (layer "B.Cu") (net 14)))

